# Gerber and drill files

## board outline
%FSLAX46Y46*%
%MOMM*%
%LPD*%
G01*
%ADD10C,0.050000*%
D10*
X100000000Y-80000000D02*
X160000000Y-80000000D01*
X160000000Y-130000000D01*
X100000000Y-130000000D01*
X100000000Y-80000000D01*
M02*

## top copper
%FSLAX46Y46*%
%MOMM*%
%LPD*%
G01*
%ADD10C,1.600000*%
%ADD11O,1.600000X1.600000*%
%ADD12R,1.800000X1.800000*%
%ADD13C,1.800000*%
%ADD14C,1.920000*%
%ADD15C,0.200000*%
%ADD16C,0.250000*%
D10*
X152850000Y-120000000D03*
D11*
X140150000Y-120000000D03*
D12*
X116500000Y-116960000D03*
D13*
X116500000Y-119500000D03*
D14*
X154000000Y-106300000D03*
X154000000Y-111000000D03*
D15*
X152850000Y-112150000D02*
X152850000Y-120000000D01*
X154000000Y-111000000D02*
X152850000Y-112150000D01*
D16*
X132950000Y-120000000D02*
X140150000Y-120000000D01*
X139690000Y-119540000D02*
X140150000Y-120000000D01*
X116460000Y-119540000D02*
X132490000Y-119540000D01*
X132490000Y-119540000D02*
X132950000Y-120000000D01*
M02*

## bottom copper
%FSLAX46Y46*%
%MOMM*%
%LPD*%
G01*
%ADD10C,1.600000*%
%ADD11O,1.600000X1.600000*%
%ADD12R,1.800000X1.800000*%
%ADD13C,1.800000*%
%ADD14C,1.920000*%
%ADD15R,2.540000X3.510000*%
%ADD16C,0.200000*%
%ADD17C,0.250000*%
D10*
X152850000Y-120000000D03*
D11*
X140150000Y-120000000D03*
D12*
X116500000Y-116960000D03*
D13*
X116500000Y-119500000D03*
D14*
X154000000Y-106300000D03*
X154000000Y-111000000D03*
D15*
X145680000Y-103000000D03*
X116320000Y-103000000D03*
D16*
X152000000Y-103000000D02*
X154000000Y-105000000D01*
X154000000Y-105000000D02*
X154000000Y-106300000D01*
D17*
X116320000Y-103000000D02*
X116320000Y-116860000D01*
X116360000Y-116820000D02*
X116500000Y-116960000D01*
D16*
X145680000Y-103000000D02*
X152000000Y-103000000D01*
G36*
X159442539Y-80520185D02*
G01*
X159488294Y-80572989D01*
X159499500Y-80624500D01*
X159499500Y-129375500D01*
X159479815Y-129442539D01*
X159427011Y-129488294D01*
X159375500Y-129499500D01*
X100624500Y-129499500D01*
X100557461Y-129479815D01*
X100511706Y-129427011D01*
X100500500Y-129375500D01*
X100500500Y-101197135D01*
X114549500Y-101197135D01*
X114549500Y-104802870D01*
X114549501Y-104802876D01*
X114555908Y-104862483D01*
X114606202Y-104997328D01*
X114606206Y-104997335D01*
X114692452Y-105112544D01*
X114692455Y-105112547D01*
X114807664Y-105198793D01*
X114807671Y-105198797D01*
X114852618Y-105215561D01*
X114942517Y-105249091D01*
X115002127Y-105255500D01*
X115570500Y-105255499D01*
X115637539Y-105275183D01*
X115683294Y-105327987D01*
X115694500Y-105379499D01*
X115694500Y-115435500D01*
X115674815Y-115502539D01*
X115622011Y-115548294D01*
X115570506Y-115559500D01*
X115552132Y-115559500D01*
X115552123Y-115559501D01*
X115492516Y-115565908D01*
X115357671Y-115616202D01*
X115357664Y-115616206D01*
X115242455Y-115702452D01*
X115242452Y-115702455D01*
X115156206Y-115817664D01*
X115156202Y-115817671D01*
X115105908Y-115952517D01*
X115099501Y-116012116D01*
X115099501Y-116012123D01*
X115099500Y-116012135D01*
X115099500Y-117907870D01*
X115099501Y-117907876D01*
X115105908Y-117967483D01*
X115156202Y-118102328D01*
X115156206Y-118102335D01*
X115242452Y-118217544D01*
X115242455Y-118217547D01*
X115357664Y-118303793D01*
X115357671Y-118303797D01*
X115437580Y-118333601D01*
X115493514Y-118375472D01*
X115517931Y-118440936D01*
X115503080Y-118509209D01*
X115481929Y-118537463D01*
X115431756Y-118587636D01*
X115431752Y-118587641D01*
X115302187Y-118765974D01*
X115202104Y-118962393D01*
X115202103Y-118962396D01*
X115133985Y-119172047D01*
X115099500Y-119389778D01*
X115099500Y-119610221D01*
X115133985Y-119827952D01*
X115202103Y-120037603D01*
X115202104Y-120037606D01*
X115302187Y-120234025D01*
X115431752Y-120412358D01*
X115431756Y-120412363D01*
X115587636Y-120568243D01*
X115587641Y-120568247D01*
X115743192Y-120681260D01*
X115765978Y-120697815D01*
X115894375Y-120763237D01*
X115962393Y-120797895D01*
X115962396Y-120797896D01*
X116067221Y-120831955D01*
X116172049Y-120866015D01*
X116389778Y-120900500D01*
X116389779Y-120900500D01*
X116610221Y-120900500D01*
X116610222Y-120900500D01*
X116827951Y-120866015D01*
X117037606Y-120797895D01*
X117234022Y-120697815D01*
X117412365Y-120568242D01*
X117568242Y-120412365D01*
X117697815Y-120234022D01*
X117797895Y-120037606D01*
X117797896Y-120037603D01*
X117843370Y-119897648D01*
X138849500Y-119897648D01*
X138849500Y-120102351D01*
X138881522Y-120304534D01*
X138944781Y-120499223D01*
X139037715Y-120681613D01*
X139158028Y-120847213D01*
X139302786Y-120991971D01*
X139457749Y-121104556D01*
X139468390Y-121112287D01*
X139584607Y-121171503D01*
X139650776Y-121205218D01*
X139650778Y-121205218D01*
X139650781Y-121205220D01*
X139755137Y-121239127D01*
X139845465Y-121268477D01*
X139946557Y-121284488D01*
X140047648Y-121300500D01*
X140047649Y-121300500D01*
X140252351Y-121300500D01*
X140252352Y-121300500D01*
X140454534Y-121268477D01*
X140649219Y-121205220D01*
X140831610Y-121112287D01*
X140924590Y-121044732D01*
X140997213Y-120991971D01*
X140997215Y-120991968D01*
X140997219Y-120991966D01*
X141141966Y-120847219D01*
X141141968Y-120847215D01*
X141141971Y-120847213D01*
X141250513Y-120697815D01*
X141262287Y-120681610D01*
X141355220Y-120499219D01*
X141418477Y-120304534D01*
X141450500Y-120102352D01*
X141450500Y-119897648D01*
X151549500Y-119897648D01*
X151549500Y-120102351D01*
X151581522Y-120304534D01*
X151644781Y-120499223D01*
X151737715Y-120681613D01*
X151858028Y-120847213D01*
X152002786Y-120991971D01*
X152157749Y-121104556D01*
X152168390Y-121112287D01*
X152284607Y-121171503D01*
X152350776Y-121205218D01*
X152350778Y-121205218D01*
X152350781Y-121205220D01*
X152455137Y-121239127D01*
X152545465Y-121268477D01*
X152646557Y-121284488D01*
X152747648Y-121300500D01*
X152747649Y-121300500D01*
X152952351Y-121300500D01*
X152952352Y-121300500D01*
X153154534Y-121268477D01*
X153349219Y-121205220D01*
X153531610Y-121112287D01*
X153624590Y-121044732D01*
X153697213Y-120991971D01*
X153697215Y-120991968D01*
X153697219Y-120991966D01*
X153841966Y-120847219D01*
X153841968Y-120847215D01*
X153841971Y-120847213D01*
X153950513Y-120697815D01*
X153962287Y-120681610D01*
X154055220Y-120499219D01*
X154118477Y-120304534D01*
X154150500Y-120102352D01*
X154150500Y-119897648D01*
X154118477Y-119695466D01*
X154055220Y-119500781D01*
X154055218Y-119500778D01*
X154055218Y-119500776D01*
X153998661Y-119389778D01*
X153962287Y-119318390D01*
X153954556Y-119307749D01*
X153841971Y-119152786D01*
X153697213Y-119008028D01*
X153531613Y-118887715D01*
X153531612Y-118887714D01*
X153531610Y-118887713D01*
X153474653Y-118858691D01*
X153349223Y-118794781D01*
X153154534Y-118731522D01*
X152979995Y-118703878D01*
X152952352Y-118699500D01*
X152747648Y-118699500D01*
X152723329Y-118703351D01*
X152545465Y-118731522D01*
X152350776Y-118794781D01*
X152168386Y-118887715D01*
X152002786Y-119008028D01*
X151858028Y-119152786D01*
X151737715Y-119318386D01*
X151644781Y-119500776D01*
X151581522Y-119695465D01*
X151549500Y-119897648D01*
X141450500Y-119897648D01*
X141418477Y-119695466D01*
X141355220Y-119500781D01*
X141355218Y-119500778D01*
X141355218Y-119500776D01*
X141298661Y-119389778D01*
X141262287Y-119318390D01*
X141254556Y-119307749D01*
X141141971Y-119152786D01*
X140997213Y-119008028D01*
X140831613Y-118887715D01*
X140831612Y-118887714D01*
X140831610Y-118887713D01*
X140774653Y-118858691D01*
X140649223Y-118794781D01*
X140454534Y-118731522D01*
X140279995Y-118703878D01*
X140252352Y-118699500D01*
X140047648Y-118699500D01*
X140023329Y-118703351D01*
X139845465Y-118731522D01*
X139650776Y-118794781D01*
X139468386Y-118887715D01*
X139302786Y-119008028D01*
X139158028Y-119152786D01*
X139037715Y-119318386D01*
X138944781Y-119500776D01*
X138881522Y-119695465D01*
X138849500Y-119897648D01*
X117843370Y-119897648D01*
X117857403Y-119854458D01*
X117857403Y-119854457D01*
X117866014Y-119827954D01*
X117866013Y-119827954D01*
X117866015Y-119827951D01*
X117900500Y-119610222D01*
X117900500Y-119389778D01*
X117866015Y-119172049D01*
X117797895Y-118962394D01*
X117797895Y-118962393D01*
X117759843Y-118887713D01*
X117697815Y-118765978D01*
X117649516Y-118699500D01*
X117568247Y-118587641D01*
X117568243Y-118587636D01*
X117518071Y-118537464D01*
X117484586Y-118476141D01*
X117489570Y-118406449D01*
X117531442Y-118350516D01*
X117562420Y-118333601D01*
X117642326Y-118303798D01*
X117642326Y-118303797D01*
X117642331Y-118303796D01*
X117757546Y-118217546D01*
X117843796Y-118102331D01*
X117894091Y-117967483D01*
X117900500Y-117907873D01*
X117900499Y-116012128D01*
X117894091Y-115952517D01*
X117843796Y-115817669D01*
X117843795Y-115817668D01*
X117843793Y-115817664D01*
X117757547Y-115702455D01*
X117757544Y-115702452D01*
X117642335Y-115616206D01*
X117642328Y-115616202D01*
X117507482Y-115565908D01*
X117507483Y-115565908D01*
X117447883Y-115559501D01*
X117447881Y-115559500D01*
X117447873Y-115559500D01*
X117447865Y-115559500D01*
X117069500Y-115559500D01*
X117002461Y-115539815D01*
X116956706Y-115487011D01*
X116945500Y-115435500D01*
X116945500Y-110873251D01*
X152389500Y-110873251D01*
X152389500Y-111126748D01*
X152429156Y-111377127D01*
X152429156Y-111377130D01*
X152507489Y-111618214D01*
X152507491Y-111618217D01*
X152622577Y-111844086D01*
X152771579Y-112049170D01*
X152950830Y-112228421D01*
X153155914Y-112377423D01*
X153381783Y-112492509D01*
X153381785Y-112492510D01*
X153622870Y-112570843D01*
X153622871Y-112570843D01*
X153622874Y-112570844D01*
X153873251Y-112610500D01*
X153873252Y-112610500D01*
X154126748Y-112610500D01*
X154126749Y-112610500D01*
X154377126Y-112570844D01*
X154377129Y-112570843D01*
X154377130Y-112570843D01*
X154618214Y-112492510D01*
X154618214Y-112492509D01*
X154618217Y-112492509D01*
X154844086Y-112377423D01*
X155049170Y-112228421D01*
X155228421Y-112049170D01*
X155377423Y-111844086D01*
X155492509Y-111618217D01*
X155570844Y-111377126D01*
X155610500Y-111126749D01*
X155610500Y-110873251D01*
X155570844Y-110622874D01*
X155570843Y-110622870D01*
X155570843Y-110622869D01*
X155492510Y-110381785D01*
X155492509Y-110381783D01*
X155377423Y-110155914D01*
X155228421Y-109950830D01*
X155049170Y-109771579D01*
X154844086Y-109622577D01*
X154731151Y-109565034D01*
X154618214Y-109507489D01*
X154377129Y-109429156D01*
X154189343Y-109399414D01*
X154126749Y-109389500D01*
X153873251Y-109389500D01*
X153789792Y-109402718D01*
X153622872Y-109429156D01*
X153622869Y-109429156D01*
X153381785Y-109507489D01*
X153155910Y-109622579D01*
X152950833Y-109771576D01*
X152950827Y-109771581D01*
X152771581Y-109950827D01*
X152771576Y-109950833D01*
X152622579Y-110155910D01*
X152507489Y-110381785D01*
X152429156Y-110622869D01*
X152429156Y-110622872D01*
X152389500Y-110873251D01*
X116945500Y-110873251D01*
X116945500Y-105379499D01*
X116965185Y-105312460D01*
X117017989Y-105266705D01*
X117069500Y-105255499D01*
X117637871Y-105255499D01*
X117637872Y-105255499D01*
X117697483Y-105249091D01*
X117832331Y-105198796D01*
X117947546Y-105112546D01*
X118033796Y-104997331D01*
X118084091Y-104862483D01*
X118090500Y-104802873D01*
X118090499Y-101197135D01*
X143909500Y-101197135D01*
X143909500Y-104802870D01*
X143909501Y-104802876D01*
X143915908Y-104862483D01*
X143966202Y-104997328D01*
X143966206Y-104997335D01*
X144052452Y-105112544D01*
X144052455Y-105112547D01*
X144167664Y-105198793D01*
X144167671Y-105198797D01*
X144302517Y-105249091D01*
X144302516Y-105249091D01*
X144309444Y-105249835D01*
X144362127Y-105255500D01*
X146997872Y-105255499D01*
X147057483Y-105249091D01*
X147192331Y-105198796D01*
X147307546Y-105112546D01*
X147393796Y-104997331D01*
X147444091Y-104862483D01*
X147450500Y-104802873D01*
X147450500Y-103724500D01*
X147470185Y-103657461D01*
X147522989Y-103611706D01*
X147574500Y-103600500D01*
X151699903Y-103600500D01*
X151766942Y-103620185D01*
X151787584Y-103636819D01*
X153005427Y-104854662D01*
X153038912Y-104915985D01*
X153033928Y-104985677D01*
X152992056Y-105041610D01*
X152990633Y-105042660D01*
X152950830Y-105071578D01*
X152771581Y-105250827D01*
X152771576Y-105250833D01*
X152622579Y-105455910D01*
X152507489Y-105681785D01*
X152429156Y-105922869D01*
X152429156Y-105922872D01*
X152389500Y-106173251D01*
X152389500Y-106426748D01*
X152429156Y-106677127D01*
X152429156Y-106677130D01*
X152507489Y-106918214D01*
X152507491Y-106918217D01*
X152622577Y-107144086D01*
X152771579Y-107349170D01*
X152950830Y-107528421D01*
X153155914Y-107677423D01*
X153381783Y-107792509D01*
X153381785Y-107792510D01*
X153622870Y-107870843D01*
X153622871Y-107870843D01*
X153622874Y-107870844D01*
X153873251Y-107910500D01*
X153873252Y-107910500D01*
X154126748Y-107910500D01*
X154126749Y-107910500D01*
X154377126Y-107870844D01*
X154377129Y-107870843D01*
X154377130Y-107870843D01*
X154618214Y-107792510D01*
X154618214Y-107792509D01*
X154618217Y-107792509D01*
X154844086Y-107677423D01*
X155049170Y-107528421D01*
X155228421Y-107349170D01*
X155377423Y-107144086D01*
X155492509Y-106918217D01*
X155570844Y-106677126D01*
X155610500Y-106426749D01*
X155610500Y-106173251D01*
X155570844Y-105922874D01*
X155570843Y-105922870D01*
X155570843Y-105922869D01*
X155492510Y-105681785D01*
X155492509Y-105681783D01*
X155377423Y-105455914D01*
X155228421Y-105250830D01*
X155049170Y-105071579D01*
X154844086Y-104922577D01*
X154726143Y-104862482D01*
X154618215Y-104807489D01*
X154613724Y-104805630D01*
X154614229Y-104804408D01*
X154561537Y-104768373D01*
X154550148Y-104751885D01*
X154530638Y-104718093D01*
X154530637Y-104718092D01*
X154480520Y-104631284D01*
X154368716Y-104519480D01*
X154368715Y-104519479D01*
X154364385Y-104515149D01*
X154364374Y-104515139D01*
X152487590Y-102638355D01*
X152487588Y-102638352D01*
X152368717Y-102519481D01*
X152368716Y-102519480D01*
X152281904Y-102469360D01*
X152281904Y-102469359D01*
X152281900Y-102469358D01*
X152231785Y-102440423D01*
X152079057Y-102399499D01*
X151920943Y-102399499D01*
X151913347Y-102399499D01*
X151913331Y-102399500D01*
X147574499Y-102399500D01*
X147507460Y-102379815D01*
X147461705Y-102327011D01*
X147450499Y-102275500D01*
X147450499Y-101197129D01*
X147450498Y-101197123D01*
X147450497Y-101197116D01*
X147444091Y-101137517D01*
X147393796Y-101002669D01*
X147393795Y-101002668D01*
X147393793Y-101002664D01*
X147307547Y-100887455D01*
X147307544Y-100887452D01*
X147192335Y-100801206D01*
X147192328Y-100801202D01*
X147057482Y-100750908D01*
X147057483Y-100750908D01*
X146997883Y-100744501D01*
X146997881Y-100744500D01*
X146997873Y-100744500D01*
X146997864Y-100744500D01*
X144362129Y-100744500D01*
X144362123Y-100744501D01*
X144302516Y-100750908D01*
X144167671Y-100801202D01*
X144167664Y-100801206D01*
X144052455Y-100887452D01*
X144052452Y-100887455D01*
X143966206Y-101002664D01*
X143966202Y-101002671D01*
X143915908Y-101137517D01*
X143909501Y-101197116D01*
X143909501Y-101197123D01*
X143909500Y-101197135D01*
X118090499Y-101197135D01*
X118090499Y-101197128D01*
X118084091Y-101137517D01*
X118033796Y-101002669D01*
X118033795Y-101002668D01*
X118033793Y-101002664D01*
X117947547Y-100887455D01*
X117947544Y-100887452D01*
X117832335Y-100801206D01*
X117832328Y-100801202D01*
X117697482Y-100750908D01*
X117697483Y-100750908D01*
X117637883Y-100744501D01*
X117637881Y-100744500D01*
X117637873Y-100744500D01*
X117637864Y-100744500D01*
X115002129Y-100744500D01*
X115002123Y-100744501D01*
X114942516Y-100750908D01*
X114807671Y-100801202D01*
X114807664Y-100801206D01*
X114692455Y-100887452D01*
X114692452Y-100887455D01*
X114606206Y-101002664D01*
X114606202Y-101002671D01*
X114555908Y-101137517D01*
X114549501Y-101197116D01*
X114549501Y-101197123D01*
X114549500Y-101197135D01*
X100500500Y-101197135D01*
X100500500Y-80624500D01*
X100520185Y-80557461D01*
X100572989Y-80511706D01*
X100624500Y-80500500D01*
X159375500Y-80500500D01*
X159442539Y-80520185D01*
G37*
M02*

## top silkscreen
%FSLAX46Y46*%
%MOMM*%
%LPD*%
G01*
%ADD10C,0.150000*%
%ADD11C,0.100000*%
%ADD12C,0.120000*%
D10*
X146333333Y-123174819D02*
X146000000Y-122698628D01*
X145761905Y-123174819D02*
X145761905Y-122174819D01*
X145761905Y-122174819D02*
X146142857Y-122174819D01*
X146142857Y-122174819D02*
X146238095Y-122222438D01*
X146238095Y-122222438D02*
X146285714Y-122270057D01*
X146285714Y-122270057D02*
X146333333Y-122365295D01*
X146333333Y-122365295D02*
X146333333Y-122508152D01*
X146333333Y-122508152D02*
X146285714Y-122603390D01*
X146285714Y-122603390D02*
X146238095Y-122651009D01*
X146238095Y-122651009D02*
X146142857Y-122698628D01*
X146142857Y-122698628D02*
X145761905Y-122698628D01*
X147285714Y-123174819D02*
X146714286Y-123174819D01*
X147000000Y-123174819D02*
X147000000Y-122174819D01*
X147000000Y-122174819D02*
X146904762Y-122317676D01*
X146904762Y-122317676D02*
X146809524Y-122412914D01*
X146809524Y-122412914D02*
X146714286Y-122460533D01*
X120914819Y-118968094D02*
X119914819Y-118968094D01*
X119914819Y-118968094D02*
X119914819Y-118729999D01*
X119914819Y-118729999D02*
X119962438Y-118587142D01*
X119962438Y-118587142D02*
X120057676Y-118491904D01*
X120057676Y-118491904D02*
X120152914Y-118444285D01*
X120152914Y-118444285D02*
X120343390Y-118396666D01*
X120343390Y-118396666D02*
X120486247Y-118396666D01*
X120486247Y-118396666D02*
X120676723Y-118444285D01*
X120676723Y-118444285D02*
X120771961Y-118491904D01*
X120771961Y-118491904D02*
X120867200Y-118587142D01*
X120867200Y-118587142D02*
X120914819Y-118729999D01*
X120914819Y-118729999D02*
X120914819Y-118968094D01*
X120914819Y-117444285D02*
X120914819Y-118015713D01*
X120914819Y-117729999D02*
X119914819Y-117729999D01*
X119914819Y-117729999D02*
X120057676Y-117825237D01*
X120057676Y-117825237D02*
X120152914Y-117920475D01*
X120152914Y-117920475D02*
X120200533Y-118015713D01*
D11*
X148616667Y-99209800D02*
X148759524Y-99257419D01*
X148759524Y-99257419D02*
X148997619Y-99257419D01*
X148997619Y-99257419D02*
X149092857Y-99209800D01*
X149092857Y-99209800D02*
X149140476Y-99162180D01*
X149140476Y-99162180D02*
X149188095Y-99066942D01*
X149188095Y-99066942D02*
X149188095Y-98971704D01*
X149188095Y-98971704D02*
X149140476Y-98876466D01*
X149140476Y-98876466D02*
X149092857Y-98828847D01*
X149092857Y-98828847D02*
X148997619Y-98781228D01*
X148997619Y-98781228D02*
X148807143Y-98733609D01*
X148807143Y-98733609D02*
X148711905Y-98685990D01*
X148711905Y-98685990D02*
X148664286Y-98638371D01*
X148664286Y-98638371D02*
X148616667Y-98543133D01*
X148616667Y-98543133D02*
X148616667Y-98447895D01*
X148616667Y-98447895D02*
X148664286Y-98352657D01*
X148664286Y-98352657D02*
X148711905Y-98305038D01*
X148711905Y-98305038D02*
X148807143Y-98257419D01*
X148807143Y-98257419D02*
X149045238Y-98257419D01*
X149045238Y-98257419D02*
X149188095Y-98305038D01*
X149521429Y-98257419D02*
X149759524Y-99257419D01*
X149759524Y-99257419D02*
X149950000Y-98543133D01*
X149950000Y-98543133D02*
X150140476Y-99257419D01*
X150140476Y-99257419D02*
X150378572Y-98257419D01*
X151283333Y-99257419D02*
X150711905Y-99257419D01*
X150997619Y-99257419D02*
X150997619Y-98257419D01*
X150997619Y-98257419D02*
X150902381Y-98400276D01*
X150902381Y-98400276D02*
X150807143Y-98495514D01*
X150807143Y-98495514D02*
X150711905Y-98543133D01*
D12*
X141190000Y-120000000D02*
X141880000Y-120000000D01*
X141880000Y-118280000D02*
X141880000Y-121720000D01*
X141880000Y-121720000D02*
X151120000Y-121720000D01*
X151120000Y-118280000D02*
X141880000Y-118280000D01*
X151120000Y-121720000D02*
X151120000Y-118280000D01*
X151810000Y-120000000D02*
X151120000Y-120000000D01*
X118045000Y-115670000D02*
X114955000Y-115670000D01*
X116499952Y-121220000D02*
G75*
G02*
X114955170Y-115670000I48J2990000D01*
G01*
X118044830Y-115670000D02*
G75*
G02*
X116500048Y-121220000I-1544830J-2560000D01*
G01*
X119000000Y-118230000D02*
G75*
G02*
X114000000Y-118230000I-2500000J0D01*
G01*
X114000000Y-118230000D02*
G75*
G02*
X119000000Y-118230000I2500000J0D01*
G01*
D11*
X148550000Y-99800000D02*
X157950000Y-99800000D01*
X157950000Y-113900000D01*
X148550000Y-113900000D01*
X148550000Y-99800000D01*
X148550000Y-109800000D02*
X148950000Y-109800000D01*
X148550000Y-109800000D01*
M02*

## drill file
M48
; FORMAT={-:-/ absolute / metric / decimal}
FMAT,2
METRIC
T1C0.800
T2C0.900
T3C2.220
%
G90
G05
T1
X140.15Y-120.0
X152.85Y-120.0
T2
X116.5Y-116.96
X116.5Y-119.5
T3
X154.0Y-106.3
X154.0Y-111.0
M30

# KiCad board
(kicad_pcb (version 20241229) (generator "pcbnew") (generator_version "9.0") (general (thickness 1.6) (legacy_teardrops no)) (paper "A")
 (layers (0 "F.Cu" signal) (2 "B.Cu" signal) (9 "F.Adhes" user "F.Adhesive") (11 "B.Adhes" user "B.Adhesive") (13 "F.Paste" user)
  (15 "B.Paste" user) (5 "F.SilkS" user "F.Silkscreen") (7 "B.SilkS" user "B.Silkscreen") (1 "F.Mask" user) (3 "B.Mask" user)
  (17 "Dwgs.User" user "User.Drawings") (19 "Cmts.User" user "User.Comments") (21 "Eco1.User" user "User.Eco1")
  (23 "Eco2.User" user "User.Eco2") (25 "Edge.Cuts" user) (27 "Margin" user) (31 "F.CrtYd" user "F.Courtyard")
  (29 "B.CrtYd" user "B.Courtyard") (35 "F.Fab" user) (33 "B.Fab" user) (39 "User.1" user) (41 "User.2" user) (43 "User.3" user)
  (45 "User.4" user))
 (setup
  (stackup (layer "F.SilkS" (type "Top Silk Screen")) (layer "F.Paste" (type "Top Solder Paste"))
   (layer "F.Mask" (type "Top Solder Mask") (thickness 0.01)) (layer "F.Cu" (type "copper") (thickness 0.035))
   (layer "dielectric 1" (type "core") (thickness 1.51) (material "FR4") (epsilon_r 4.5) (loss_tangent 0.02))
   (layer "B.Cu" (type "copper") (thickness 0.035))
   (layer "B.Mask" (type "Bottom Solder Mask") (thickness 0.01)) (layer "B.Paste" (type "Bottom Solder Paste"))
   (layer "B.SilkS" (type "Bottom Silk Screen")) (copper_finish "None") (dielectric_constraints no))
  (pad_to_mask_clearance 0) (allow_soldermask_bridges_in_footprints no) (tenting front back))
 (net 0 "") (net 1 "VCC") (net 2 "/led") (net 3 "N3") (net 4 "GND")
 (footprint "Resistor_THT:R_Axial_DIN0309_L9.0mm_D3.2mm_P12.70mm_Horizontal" (layer "F.Cu") (at 152.85 120 180)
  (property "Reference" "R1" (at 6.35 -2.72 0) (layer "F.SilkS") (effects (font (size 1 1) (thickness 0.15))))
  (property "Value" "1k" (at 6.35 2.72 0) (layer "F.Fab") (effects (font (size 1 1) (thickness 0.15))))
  (fp_line (start 11.66 0) (end 10.97 0) (stroke (width 0.12) (type solid)) (layer "F.SilkS"))
  (fp_line (start 10.97 1.72) (end 10.97 -1.72) (stroke (width 0.12) (type solid)) (layer "F.SilkS"))
  (fp_line (start 10.97 -1.72) (end 1.73 -1.72) (stroke (width 0.12) (type solid)) (layer "F.SilkS"))
  (fp_line (start 1.73 1.72) (end 10.97 1.72) (stroke (width 0.12) (type solid)) (layer "F.SilkS"))
  (fp_line (start 1.73 -1.72) (end 1.73 1.72) (stroke (width 0.12) (type solid)) (layer "F.SilkS"))
  (fp_line (start 1.04 0) (end 1.73 0) (stroke (width 0.12) (type solid)) (layer "F.SilkS"))
  (pad "1" thru_hole circle (at 0 0 180) (size 1.6 1.6) (drill 0.8) (layers "*.Cu" "*.Mask") (remove_unused_layers no) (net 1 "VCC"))
  (pad "2" thru_hole oval (at 12.7 0 180) (size 1.6 1.6) (drill 0.8) (layers "*.Cu" "*.Mask") (remove_unused_layers no) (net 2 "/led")))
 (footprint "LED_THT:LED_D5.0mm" (layer "F.Cu") (at 116.5 116.96 -90)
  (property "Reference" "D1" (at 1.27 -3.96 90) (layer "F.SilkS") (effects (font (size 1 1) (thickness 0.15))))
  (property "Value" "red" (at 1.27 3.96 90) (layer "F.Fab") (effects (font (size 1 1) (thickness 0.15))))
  (fp_line (start -1.29 -1.545) (end -1.29 1.545) (stroke (width 0.12) (type solid)) (layer "F.SilkS"))
  (fp_arc (start 4.26 0.000048) (mid 2.071756 2.880501) (end -1.29 1.54483) (stroke (width 0.12) (type solid)) (layer "F.SilkS"))
  (fp_arc (start -1.29 -1.54483) (mid 2.071756 -2.880501) (end 4.26 -0.000048) (stroke (width 0.12) (type solid)) (layer "F.SilkS"))
  (fp_circle (center 1.27 0) (end 3.77 0) (stroke (width 0.12) (type solid)) (fill no) (layer "F.SilkS"))
  (pad "1" thru_hole rect (at 0 0 270) (size 1.8 1.8) (drill 0.9) (layers "*.Cu" "*.Mask") (remove_unused_layers no) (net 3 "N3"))
  (pad "2" thru_hole circle (at 2.54 0 270) (size 1.8 1.8) (drill 0.9) (layers "*.Cu" "*.Mask") (remove_unused_layers no) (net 2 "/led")))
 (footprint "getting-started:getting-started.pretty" (layer "F.Cu") (at 154 101.6)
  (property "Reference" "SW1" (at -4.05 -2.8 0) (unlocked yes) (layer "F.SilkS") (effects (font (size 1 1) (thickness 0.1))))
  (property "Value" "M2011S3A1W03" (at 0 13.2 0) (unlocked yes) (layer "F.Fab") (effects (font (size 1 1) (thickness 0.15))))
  (fp_rect (start -5.45 -1.8) (end 3.95 12.3) (stroke (width 0.1) (type default)) (fill no) (layer "F.SilkS"))
  (fp_rect (start -5.45 8.2) (end -5.05 8.2) (stroke (width 0.1) (type default)) (fill no) (layer "F.SilkS"))
  (pad "2" thru_hole circle (at 0 4.7) (size 1.92 1.92) (drill 2.22) (layers "*.Cu" "*.Mask") (remove_unused_layers no) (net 3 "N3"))
  (pad "3" thru_hole circle (at 0 9.4) (size 1.92 1.92) (drill 2.22) (layers "*.Cu" "*.Mask") (remove_unused_layers no) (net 1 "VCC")))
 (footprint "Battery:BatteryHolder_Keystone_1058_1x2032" (layer "B.Cu") (at 131 103 180)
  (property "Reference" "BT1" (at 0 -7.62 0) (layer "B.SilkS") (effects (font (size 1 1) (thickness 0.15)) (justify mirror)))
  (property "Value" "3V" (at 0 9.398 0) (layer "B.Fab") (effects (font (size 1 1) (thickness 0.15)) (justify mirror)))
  (pad "1" smd rect (at -14.68 0 180) (size 2.54 3.51) (layers "B.Cu" "B.Mask" "B.Paste") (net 3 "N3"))
  (pad "2" smd rect (at 14.68 0 180) (size 2.54 3.51) (layers "B.Cu" "B.Mask" "B.Paste") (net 3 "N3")))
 (gr_rect (start 100 80) (end 160 130) (stroke (width 0.05) (type default)) (fill no) (layer "Edge.Cuts"))
 (segment (start 152.85 112.15) (end 152.85 120) (width 0.2) (layer "F.Cu") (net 1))
 (segment (start 154 111) (end 152.85 112.15) (width 0.2) (layer "F.Cu") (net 1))
 (segment (start 132.95 120) (end 140.15 120) (width 0.25) (layer "F.Cu") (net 2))
 (segment (start 139.69 119.54) (end 140.15 120) (width 0.25) (layer "F.Cu") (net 2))
 (segment (start 116.46 119.54) (end 132.49 119.54) (width 0.25) (layer "F.Cu") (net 2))
 (segment (start 132.49 119.54) (end 132.95 120) (width 0.25) (layer "F.Cu") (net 2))
 (segment (start 152 103) (end 154 105) (width 0.2) (layers "B.Cu" "B.Mask") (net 3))
 (segment (start 154 105) (end 154 106.3) (width 0.2) (layer "B.Cu") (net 3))
 (segment (start 116.32 103) (end 116.32 116.86) (width 0.25) (layer "B.Cu") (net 3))
 (segment (start 116.36 116.82) (end 116.5 116.96) (width 0.25) (layer "B.Cu") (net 3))
 (segment (start 145.68 103) (end 152 103) (width 0.2) (layers "B.Cu" "B.Mask") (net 3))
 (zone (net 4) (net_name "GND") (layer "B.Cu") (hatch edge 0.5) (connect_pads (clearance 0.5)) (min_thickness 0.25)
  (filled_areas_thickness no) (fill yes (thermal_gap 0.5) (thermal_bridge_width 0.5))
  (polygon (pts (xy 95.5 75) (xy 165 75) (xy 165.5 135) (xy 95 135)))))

